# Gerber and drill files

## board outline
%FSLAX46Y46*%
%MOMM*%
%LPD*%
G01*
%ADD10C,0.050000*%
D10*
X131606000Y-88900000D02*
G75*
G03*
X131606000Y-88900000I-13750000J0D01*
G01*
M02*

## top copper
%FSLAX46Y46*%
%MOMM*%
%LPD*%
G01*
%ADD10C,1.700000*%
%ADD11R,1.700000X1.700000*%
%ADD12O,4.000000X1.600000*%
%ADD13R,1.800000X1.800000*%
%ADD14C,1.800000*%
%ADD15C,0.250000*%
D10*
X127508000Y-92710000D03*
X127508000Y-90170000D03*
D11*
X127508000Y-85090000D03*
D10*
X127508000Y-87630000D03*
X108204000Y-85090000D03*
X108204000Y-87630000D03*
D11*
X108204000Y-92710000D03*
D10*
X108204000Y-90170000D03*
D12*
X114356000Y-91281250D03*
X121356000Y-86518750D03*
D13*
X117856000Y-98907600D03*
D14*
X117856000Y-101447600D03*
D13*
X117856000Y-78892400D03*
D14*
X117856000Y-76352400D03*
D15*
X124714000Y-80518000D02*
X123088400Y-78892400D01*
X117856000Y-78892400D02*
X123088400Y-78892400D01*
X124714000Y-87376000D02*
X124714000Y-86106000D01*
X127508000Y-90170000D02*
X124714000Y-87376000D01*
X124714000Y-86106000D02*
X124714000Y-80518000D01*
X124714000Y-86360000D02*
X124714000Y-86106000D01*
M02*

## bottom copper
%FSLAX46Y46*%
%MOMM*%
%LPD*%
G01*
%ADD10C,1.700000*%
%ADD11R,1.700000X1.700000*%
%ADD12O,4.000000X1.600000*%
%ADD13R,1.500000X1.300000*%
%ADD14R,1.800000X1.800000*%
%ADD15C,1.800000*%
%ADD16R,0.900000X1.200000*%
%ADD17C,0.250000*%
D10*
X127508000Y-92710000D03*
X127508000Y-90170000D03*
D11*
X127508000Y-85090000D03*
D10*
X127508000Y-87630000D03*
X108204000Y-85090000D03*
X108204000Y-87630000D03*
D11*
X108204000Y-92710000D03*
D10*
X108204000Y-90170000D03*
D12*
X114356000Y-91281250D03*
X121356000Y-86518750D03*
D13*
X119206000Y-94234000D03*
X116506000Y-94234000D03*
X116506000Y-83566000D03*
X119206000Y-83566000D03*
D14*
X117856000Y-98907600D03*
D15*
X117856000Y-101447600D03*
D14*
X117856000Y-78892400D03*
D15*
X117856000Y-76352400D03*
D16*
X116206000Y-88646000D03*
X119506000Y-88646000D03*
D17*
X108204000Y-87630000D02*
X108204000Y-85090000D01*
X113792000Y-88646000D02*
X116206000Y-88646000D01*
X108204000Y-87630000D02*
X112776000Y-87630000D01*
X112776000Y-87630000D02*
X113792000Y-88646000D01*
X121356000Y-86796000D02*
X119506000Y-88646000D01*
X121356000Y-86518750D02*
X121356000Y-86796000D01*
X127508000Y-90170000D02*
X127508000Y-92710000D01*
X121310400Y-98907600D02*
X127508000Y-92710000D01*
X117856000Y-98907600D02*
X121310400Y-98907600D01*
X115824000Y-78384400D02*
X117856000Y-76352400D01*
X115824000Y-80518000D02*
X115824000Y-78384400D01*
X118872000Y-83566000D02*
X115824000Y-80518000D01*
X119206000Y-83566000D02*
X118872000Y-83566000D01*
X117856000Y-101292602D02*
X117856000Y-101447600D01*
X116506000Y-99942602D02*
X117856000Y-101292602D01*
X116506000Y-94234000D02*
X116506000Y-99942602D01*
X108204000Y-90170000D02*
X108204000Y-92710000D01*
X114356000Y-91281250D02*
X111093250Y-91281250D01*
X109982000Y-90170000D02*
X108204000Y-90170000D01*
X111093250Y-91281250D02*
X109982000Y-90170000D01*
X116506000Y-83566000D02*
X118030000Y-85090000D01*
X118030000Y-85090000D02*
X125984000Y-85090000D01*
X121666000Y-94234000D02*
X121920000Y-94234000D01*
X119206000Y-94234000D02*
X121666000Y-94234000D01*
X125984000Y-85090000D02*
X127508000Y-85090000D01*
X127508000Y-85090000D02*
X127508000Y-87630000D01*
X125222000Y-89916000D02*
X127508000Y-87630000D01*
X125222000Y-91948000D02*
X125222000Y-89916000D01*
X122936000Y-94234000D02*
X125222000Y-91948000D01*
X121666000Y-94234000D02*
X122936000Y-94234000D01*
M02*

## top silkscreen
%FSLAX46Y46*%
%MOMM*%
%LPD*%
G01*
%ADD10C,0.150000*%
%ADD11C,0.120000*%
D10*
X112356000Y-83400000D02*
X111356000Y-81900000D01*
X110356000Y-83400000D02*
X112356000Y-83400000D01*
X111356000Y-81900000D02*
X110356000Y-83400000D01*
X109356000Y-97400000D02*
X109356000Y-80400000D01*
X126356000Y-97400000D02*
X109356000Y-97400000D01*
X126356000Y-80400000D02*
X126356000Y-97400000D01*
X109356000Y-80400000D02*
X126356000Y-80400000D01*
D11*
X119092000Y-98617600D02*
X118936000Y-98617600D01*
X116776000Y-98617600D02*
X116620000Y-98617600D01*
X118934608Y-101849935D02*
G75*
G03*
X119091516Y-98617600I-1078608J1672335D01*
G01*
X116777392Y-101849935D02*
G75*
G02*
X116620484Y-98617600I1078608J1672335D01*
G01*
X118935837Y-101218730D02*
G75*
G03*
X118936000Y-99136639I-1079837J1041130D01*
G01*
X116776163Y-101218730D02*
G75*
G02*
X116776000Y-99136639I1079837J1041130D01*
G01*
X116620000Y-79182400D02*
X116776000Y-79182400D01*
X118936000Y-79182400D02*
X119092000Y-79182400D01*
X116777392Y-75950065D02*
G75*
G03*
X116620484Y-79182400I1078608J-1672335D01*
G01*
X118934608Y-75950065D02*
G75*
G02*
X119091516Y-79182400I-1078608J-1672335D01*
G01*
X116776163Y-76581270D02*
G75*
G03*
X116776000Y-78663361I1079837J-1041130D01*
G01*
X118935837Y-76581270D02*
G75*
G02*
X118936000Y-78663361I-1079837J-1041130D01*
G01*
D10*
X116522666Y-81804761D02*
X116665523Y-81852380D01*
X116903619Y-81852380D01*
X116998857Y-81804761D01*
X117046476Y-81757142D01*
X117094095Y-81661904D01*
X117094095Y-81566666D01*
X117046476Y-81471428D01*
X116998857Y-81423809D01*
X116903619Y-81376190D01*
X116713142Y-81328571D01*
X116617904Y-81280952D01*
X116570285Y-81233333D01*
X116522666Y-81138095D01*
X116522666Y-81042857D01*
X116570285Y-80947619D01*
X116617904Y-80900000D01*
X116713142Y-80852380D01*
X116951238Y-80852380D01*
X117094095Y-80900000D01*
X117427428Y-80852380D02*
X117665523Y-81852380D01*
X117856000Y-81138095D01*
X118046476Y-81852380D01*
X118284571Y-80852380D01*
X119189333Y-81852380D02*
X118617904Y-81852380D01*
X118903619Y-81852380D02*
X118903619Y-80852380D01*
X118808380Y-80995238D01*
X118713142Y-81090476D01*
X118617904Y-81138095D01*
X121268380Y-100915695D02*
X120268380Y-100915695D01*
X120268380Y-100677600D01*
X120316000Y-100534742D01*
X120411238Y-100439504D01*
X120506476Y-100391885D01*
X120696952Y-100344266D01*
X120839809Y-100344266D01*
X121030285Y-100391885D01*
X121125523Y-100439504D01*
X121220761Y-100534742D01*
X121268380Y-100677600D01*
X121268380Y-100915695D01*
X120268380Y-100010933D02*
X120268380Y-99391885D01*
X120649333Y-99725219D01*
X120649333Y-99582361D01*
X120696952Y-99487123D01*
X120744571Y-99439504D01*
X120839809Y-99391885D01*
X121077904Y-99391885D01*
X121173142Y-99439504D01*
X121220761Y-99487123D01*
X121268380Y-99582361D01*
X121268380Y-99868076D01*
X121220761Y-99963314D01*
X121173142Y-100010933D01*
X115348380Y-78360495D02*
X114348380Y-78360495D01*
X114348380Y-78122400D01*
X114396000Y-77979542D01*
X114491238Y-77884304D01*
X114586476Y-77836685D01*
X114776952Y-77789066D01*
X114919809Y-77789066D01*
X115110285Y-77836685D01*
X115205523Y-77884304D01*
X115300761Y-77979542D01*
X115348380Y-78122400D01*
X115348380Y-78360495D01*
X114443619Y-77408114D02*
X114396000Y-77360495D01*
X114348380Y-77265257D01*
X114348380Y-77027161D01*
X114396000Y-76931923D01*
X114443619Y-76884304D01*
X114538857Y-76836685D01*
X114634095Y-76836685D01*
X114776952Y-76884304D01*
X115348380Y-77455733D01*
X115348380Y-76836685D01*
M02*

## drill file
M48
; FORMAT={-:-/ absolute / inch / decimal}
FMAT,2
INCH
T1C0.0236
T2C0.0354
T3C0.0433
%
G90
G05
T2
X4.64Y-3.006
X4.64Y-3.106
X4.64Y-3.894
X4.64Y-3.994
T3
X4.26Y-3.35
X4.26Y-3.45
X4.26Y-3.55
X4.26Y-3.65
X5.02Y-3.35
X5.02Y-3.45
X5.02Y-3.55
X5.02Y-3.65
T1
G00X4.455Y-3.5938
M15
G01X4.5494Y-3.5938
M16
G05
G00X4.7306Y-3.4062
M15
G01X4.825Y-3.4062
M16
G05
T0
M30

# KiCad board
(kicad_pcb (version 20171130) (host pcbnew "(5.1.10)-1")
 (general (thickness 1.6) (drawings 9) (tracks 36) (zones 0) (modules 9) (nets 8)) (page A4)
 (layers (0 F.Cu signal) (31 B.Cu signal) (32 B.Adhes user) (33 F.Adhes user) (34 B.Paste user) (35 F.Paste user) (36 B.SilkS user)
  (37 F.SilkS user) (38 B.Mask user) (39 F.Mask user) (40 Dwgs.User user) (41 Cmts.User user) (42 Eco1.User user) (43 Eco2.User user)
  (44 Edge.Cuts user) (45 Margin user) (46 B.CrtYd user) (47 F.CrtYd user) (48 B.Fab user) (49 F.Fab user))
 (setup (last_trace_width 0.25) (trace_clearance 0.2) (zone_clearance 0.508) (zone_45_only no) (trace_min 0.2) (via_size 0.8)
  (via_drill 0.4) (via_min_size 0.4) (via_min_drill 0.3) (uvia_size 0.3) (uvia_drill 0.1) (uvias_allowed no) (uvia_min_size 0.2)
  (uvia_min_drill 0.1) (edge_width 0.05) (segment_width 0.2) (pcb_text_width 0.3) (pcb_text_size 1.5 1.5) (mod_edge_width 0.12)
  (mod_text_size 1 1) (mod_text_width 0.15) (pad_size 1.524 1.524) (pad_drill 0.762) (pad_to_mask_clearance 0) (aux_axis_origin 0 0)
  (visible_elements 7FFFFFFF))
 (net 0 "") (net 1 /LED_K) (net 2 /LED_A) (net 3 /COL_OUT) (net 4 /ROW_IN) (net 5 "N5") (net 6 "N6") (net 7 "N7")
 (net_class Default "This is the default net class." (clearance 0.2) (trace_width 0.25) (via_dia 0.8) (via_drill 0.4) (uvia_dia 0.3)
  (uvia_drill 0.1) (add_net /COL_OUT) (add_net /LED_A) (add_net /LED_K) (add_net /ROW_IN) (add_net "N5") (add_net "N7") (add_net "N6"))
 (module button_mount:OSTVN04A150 (layer B.Cu) (at 127.508 85.09 270)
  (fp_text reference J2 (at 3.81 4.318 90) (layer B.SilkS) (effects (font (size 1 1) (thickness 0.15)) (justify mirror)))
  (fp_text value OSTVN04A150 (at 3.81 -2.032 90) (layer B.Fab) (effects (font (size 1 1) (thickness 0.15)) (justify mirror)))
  (pad 4 thru_hole circle (at 7.62 0 270) (size 1.7 1.7) (drill 1.1) (layers *.Cu *.Mask) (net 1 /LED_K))
  (pad 3 thru_hole circle (at 5.08 0 270) (size 1.7 1.7) (drill 1.1) (layers *.Cu *.Mask) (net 1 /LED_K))
  (pad 1 thru_hole rect (at 0 0 270) (size 1.7 1.7) (drill 1.1) (layers *.Cu *.Mask) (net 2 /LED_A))
  (pad 2 thru_hole circle (at 2.54 0 270) (size 1.7 1.7) (drill 1.1) (layers *.Cu *.Mask) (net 2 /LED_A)))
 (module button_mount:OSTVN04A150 (layer B.Cu) (at 108.204 92.71 90)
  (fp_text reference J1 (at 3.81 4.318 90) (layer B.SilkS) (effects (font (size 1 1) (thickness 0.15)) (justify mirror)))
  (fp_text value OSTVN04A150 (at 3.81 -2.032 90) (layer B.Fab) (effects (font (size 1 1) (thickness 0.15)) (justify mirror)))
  (pad 4 thru_hole circle (at 7.62 0 90) (size 1.7 1.7) (drill 1.1) (layers *.Cu *.Mask) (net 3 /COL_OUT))
  (pad 3 thru_hole circle (at 5.08 0 90) (size 1.7 1.7) (drill 1.1) (layers *.Cu *.Mask) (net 3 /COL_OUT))
  (pad 1 thru_hole rect (at 0 0 90) (size 1.7 1.7) (drill 1.1) (layers *.Cu *.Mask) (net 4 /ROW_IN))
  (pad 2 thru_hole circle (at 2.54 0 90) (size 1.7 1.7) (drill 1.1) (layers *.Cu *.Mask) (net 4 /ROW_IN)))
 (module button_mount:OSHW (layer B.Cu) (at 112.268 97.282 180)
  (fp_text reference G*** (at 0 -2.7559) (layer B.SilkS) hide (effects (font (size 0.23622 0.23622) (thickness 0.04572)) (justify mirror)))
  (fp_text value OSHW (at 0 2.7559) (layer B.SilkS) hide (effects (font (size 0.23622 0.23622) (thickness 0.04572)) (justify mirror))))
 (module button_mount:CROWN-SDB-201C (layer F.Cu) (at 117.856 88.9)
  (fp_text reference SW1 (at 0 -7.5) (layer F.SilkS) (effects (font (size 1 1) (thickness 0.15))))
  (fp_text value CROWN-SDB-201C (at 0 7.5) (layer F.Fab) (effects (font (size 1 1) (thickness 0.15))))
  (fp_line (start -5.5 -5.5) (end -6.5 -7) (layer F.SilkS) (width 0.15))
  (fp_line (start -7.5 -5.5) (end -5.5 -5.5) (layer F.SilkS) (width 0.15))
  (fp_line (start -6.5 -7) (end -7.5 -5.5) (layer F.SilkS) (width 0.15))
  (fp_line (start -8.5 8.5) (end -8.5 -8.5) (layer F.SilkS) (width 0.15))
  (fp_line (start 8.5 8.5) (end -8.5 8.5) (layer F.SilkS) (width 0.15))
  (fp_line (start 8.5 -8.5) (end 8.5 8.5) (layer F.SilkS) (width 0.15))
  (fp_line (start -8.5 -8.5) (end 8.5 -8.5) (layer F.SilkS) (width 0.15))
  (pad 2 thru_hole oval (at -3.5 2.38125) (size 4 1.6) (drill oval 3 0.6) (layers *.Cu *.Mask) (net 4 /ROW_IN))
  (pad 1 thru_hole oval (at 3.5 -2.38125) (size 4 1.6) (drill oval 3 0.6) (layers *.Cu *.Mask) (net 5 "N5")))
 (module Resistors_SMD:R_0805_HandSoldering (layer B.Cu) (at 117.856 94.234 180)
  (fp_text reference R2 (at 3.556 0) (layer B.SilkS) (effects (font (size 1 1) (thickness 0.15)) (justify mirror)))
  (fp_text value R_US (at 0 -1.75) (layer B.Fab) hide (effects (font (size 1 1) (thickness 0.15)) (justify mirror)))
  (pad 1 smd rect (at -1.35 0 180) (size 1.5 1.3) (layers B.Cu B.Paste B.Mask) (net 2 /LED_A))
  (pad 2 smd rect (at 1.35 0 180) (size 1.5 1.3) (layers B.Cu B.Paste B.Mask) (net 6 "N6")))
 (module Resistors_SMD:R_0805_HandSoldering (layer B.Cu) (at 117.856 83.566)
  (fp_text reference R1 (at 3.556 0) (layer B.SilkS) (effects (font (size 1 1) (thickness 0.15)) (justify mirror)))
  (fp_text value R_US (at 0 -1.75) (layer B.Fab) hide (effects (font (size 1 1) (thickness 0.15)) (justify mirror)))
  (pad 1 smd rect (at -1.35 0) (size 1.5 1.3) (layers B.Cu B.Paste B.Mask) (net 2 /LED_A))
  (pad 2 smd rect (at 1.35 0) (size 1.5 1.3) (layers B.Cu B.Paste B.Mask) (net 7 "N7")))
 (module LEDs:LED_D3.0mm (layer F.Cu) (at 117.856 98.9076 270)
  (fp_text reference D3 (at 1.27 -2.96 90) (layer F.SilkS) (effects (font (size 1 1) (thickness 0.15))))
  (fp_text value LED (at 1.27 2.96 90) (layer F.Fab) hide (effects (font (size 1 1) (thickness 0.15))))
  (fp_line (start -0.29 -1.236) (end -0.29 -1.08) (layer F.SilkS) (width 0.12))
  (fp_line (start -0.29 1.08) (end -0.29 1.236) (layer F.SilkS) (width 0.12))
  (fp_arc (start 1.27 0) (end -0.29 -1.235516) (angle 108.8) (layer F.SilkS) (width 0.12))
  (fp_arc (start 1.27 0) (end -0.29 1.235516) (angle -108.8) (layer F.SilkS) (width 0.12))
  (fp_arc (start 1.27 0) (end 0.229039 -1.08) (angle 87.9) (layer F.SilkS) (width 0.12))
  (fp_arc (start 1.27 0) (end 0.229039 1.08) (angle -87.9) (layer F.SilkS) (width 0.12))
  (pad 1 thru_hole rect (at 0 0 270) (size 1.8 1.8) (drill 0.9) (layers *.Cu *.Mask) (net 1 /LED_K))
  (pad 2 thru_hole circle (at 2.54 0 270) (size 1.8 1.8) (drill 0.9) (layers *.Cu *.Mask) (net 6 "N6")))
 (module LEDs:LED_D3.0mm (layer F.Cu) (at 117.856 78.8924 90)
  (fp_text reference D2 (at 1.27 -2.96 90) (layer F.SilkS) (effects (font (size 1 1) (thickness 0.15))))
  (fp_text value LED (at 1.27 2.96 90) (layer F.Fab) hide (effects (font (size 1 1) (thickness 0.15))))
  (fp_line (start -0.29 -1.236) (end -0.29 -1.08) (layer F.SilkS) (width 0.12))
  (fp_line (start -0.29 1.08) (end -0.29 1.236) (layer F.SilkS) (width 0.12))
  (fp_arc (start 1.27 0) (end -0.29 -1.235516) (angle 108.8) (layer F.SilkS) (width 0.12))
  (fp_arc (start 1.27 0) (end -0.29 1.235516) (angle -108.8) (layer F.SilkS) (width 0.12))
  (fp_arc (start 1.27 0) (end 0.229039 -1.08) (angle 87.9) (layer F.SilkS) (width 0.12))
  (fp_arc (start 1.27 0) (end 0.229039 1.08) (angle -87.9) (layer F.SilkS) (width 0.12))
  (pad 1 thru_hole rect (at 0 0 90) (size 1.8 1.8) (drill 0.9) (layers *.Cu *.Mask) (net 1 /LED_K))
  (pad 2 thru_hole circle (at 2.54 0 90) (size 1.8 1.8) (drill 0.9) (layers *.Cu *.Mask) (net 7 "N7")))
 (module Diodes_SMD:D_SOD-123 (layer B.Cu) (at 117.856 88.646)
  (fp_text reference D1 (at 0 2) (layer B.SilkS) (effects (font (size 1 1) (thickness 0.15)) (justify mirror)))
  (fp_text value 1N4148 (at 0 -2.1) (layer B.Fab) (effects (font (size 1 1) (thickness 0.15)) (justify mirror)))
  (pad 1 smd rect (at -1.65 0) (size 0.9 1.2) (layers B.Cu B.Paste B.Mask) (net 3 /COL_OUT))
  (pad 2 smd rect (at 1.65 0) (size 0.9 1.2) (layers B.Cu B.Paste B.Mask) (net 5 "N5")))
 (gr_circle (center 117.856 88.9) (end 131.606 88.9) (layer Edge.Cuts) (width 0.05))
 (segment (start 108.204 87.63) (end 108.204 85.09) (width 0.25) (layer B.Cu) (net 3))
 (segment (start 113.792 88.646) (end 116.206 88.646) (width 0.25) (layer B.Cu) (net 3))
 (segment (start 108.204 87.63) (end 112.776 87.63) (width 0.25) (layer B.Cu) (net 3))
 (segment (start 112.776 87.63) (end 113.792 88.646) (width 0.25) (layer B.Cu) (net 3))
 (segment (start 121.356 86.796) (end 119.506 88.646) (width 0.25) (layer B.Cu) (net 5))
 (segment (start 121.356 86.51875) (end 121.356 86.796) (width 0.25) (layer B.Cu) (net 5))
 (segment (start 124.714 80.518) (end 123.0884 78.8924) (width 0.25) (layer F.Cu) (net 1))
 (segment (start 117.856 78.8924) (end 123.0884 78.8924) (width 0.25) (layer F.Cu) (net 1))
 (segment (start 127.508 90.17) (end 127.508 92.71) (width 0.25) (layer B.Cu) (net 1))
 (segment (start 121.3104 98.9076) (end 127.508 92.71) (width 0.25) (layer B.Cu) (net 1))
 (segment (start 117.856 98.9076) (end 121.3104 98.9076) (width 0.25) (layer B.Cu) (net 1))
 (segment (start 124.714 87.376) (end 124.714 86.106) (width 0.25) (layer F.Cu) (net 1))
 (segment (start 127.508 90.17) (end 124.714 87.376) (width 0.25) (layer F.Cu) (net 1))
 (segment (start 124.714 86.106) (end 124.714 80.518) (width 0.25) (layer F.Cu) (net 1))
 (segment (start 124.714 86.36) (end 124.714 86.106) (width 0.25) (layer F.Cu) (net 1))
 (segment (start 115.824 78.3844) (end 117.856 76.3524) (width 0.25) (layer B.Cu) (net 7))
 (segment (start 115.824 80.518) (end 115.824 78.3844) (width 0.25) (layer B.Cu) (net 7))
 (segment (start 118.872 83.566) (end 115.824 80.518) (width 0.25) (layer B.Cu) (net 7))
 (segment (start 119.206 83.566) (end 118.872 83.566) (width 0.25) (layer B.Cu) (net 7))
 (segment (start 117.856 101.292602) (end 117.856 101.4476) (width 0.25) (layer B.Cu) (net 6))
 (segment (start 116.506 99.942602) (end 117.856 101.292602) (width 0.25) (layer B.Cu) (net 6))
 (segment (start 116.506 94.234) (end 116.506 99.942602) (width 0.25) (layer B.Cu) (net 6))
 (segment (start 108.204 90.17) (end 108.204 92.71) (width 0.25) (layer B.Cu) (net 4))
 (segment (start 114.356 91.28125) (end 111.09325 91.28125) (width 0.25) (layer B.Cu) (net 4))
 (segment (start 109.982 90.17) (end 108.204 90.17) (width 0.25) (layer B.Cu) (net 4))
 (segment (start 111.09325 91.28125) (end 109.982 90.17) (width 0.25) (layer B.Cu) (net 4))
 (segment (start 116.506 83.566) (end 118.03 85.09) (width 0.25) (layer B.Cu) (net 2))
 (segment (start 118.03 85.09) (end 125.984 85.09) (width 0.25) (layer B.Cu) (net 2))
 (segment (start 121.666 94.234) (end 121.92 94.234) (width 0.25) (layer B.Cu) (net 2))
 (segment (start 119.206 94.234) (end 121.666 94.234) (width 0.25) (layer B.Cu) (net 2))
 (segment (start 125.984 85.09) (end 127.508 85.09) (width 0.25) (layer B.Cu) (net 2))
 (segment (start 127.508 85.09) (end 127.508 87.63) (width 0.25) (layer B.Cu) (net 2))
 (segment (start 125.222 89.916) (end 127.508 87.63) (width 0.25) (layer B.Cu) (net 2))
 (segment (start 125.222 91.948) (end 125.222 89.916) (width 0.25) (layer B.Cu) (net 2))
 (segment (start 122.936 94.234) (end 125.222 91.948) (width 0.25) (layer B.Cu) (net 2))
 (segment (start 121.666 94.234) (end 122.936 94.234) (width 0.25) (layer B.Cu) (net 2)))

